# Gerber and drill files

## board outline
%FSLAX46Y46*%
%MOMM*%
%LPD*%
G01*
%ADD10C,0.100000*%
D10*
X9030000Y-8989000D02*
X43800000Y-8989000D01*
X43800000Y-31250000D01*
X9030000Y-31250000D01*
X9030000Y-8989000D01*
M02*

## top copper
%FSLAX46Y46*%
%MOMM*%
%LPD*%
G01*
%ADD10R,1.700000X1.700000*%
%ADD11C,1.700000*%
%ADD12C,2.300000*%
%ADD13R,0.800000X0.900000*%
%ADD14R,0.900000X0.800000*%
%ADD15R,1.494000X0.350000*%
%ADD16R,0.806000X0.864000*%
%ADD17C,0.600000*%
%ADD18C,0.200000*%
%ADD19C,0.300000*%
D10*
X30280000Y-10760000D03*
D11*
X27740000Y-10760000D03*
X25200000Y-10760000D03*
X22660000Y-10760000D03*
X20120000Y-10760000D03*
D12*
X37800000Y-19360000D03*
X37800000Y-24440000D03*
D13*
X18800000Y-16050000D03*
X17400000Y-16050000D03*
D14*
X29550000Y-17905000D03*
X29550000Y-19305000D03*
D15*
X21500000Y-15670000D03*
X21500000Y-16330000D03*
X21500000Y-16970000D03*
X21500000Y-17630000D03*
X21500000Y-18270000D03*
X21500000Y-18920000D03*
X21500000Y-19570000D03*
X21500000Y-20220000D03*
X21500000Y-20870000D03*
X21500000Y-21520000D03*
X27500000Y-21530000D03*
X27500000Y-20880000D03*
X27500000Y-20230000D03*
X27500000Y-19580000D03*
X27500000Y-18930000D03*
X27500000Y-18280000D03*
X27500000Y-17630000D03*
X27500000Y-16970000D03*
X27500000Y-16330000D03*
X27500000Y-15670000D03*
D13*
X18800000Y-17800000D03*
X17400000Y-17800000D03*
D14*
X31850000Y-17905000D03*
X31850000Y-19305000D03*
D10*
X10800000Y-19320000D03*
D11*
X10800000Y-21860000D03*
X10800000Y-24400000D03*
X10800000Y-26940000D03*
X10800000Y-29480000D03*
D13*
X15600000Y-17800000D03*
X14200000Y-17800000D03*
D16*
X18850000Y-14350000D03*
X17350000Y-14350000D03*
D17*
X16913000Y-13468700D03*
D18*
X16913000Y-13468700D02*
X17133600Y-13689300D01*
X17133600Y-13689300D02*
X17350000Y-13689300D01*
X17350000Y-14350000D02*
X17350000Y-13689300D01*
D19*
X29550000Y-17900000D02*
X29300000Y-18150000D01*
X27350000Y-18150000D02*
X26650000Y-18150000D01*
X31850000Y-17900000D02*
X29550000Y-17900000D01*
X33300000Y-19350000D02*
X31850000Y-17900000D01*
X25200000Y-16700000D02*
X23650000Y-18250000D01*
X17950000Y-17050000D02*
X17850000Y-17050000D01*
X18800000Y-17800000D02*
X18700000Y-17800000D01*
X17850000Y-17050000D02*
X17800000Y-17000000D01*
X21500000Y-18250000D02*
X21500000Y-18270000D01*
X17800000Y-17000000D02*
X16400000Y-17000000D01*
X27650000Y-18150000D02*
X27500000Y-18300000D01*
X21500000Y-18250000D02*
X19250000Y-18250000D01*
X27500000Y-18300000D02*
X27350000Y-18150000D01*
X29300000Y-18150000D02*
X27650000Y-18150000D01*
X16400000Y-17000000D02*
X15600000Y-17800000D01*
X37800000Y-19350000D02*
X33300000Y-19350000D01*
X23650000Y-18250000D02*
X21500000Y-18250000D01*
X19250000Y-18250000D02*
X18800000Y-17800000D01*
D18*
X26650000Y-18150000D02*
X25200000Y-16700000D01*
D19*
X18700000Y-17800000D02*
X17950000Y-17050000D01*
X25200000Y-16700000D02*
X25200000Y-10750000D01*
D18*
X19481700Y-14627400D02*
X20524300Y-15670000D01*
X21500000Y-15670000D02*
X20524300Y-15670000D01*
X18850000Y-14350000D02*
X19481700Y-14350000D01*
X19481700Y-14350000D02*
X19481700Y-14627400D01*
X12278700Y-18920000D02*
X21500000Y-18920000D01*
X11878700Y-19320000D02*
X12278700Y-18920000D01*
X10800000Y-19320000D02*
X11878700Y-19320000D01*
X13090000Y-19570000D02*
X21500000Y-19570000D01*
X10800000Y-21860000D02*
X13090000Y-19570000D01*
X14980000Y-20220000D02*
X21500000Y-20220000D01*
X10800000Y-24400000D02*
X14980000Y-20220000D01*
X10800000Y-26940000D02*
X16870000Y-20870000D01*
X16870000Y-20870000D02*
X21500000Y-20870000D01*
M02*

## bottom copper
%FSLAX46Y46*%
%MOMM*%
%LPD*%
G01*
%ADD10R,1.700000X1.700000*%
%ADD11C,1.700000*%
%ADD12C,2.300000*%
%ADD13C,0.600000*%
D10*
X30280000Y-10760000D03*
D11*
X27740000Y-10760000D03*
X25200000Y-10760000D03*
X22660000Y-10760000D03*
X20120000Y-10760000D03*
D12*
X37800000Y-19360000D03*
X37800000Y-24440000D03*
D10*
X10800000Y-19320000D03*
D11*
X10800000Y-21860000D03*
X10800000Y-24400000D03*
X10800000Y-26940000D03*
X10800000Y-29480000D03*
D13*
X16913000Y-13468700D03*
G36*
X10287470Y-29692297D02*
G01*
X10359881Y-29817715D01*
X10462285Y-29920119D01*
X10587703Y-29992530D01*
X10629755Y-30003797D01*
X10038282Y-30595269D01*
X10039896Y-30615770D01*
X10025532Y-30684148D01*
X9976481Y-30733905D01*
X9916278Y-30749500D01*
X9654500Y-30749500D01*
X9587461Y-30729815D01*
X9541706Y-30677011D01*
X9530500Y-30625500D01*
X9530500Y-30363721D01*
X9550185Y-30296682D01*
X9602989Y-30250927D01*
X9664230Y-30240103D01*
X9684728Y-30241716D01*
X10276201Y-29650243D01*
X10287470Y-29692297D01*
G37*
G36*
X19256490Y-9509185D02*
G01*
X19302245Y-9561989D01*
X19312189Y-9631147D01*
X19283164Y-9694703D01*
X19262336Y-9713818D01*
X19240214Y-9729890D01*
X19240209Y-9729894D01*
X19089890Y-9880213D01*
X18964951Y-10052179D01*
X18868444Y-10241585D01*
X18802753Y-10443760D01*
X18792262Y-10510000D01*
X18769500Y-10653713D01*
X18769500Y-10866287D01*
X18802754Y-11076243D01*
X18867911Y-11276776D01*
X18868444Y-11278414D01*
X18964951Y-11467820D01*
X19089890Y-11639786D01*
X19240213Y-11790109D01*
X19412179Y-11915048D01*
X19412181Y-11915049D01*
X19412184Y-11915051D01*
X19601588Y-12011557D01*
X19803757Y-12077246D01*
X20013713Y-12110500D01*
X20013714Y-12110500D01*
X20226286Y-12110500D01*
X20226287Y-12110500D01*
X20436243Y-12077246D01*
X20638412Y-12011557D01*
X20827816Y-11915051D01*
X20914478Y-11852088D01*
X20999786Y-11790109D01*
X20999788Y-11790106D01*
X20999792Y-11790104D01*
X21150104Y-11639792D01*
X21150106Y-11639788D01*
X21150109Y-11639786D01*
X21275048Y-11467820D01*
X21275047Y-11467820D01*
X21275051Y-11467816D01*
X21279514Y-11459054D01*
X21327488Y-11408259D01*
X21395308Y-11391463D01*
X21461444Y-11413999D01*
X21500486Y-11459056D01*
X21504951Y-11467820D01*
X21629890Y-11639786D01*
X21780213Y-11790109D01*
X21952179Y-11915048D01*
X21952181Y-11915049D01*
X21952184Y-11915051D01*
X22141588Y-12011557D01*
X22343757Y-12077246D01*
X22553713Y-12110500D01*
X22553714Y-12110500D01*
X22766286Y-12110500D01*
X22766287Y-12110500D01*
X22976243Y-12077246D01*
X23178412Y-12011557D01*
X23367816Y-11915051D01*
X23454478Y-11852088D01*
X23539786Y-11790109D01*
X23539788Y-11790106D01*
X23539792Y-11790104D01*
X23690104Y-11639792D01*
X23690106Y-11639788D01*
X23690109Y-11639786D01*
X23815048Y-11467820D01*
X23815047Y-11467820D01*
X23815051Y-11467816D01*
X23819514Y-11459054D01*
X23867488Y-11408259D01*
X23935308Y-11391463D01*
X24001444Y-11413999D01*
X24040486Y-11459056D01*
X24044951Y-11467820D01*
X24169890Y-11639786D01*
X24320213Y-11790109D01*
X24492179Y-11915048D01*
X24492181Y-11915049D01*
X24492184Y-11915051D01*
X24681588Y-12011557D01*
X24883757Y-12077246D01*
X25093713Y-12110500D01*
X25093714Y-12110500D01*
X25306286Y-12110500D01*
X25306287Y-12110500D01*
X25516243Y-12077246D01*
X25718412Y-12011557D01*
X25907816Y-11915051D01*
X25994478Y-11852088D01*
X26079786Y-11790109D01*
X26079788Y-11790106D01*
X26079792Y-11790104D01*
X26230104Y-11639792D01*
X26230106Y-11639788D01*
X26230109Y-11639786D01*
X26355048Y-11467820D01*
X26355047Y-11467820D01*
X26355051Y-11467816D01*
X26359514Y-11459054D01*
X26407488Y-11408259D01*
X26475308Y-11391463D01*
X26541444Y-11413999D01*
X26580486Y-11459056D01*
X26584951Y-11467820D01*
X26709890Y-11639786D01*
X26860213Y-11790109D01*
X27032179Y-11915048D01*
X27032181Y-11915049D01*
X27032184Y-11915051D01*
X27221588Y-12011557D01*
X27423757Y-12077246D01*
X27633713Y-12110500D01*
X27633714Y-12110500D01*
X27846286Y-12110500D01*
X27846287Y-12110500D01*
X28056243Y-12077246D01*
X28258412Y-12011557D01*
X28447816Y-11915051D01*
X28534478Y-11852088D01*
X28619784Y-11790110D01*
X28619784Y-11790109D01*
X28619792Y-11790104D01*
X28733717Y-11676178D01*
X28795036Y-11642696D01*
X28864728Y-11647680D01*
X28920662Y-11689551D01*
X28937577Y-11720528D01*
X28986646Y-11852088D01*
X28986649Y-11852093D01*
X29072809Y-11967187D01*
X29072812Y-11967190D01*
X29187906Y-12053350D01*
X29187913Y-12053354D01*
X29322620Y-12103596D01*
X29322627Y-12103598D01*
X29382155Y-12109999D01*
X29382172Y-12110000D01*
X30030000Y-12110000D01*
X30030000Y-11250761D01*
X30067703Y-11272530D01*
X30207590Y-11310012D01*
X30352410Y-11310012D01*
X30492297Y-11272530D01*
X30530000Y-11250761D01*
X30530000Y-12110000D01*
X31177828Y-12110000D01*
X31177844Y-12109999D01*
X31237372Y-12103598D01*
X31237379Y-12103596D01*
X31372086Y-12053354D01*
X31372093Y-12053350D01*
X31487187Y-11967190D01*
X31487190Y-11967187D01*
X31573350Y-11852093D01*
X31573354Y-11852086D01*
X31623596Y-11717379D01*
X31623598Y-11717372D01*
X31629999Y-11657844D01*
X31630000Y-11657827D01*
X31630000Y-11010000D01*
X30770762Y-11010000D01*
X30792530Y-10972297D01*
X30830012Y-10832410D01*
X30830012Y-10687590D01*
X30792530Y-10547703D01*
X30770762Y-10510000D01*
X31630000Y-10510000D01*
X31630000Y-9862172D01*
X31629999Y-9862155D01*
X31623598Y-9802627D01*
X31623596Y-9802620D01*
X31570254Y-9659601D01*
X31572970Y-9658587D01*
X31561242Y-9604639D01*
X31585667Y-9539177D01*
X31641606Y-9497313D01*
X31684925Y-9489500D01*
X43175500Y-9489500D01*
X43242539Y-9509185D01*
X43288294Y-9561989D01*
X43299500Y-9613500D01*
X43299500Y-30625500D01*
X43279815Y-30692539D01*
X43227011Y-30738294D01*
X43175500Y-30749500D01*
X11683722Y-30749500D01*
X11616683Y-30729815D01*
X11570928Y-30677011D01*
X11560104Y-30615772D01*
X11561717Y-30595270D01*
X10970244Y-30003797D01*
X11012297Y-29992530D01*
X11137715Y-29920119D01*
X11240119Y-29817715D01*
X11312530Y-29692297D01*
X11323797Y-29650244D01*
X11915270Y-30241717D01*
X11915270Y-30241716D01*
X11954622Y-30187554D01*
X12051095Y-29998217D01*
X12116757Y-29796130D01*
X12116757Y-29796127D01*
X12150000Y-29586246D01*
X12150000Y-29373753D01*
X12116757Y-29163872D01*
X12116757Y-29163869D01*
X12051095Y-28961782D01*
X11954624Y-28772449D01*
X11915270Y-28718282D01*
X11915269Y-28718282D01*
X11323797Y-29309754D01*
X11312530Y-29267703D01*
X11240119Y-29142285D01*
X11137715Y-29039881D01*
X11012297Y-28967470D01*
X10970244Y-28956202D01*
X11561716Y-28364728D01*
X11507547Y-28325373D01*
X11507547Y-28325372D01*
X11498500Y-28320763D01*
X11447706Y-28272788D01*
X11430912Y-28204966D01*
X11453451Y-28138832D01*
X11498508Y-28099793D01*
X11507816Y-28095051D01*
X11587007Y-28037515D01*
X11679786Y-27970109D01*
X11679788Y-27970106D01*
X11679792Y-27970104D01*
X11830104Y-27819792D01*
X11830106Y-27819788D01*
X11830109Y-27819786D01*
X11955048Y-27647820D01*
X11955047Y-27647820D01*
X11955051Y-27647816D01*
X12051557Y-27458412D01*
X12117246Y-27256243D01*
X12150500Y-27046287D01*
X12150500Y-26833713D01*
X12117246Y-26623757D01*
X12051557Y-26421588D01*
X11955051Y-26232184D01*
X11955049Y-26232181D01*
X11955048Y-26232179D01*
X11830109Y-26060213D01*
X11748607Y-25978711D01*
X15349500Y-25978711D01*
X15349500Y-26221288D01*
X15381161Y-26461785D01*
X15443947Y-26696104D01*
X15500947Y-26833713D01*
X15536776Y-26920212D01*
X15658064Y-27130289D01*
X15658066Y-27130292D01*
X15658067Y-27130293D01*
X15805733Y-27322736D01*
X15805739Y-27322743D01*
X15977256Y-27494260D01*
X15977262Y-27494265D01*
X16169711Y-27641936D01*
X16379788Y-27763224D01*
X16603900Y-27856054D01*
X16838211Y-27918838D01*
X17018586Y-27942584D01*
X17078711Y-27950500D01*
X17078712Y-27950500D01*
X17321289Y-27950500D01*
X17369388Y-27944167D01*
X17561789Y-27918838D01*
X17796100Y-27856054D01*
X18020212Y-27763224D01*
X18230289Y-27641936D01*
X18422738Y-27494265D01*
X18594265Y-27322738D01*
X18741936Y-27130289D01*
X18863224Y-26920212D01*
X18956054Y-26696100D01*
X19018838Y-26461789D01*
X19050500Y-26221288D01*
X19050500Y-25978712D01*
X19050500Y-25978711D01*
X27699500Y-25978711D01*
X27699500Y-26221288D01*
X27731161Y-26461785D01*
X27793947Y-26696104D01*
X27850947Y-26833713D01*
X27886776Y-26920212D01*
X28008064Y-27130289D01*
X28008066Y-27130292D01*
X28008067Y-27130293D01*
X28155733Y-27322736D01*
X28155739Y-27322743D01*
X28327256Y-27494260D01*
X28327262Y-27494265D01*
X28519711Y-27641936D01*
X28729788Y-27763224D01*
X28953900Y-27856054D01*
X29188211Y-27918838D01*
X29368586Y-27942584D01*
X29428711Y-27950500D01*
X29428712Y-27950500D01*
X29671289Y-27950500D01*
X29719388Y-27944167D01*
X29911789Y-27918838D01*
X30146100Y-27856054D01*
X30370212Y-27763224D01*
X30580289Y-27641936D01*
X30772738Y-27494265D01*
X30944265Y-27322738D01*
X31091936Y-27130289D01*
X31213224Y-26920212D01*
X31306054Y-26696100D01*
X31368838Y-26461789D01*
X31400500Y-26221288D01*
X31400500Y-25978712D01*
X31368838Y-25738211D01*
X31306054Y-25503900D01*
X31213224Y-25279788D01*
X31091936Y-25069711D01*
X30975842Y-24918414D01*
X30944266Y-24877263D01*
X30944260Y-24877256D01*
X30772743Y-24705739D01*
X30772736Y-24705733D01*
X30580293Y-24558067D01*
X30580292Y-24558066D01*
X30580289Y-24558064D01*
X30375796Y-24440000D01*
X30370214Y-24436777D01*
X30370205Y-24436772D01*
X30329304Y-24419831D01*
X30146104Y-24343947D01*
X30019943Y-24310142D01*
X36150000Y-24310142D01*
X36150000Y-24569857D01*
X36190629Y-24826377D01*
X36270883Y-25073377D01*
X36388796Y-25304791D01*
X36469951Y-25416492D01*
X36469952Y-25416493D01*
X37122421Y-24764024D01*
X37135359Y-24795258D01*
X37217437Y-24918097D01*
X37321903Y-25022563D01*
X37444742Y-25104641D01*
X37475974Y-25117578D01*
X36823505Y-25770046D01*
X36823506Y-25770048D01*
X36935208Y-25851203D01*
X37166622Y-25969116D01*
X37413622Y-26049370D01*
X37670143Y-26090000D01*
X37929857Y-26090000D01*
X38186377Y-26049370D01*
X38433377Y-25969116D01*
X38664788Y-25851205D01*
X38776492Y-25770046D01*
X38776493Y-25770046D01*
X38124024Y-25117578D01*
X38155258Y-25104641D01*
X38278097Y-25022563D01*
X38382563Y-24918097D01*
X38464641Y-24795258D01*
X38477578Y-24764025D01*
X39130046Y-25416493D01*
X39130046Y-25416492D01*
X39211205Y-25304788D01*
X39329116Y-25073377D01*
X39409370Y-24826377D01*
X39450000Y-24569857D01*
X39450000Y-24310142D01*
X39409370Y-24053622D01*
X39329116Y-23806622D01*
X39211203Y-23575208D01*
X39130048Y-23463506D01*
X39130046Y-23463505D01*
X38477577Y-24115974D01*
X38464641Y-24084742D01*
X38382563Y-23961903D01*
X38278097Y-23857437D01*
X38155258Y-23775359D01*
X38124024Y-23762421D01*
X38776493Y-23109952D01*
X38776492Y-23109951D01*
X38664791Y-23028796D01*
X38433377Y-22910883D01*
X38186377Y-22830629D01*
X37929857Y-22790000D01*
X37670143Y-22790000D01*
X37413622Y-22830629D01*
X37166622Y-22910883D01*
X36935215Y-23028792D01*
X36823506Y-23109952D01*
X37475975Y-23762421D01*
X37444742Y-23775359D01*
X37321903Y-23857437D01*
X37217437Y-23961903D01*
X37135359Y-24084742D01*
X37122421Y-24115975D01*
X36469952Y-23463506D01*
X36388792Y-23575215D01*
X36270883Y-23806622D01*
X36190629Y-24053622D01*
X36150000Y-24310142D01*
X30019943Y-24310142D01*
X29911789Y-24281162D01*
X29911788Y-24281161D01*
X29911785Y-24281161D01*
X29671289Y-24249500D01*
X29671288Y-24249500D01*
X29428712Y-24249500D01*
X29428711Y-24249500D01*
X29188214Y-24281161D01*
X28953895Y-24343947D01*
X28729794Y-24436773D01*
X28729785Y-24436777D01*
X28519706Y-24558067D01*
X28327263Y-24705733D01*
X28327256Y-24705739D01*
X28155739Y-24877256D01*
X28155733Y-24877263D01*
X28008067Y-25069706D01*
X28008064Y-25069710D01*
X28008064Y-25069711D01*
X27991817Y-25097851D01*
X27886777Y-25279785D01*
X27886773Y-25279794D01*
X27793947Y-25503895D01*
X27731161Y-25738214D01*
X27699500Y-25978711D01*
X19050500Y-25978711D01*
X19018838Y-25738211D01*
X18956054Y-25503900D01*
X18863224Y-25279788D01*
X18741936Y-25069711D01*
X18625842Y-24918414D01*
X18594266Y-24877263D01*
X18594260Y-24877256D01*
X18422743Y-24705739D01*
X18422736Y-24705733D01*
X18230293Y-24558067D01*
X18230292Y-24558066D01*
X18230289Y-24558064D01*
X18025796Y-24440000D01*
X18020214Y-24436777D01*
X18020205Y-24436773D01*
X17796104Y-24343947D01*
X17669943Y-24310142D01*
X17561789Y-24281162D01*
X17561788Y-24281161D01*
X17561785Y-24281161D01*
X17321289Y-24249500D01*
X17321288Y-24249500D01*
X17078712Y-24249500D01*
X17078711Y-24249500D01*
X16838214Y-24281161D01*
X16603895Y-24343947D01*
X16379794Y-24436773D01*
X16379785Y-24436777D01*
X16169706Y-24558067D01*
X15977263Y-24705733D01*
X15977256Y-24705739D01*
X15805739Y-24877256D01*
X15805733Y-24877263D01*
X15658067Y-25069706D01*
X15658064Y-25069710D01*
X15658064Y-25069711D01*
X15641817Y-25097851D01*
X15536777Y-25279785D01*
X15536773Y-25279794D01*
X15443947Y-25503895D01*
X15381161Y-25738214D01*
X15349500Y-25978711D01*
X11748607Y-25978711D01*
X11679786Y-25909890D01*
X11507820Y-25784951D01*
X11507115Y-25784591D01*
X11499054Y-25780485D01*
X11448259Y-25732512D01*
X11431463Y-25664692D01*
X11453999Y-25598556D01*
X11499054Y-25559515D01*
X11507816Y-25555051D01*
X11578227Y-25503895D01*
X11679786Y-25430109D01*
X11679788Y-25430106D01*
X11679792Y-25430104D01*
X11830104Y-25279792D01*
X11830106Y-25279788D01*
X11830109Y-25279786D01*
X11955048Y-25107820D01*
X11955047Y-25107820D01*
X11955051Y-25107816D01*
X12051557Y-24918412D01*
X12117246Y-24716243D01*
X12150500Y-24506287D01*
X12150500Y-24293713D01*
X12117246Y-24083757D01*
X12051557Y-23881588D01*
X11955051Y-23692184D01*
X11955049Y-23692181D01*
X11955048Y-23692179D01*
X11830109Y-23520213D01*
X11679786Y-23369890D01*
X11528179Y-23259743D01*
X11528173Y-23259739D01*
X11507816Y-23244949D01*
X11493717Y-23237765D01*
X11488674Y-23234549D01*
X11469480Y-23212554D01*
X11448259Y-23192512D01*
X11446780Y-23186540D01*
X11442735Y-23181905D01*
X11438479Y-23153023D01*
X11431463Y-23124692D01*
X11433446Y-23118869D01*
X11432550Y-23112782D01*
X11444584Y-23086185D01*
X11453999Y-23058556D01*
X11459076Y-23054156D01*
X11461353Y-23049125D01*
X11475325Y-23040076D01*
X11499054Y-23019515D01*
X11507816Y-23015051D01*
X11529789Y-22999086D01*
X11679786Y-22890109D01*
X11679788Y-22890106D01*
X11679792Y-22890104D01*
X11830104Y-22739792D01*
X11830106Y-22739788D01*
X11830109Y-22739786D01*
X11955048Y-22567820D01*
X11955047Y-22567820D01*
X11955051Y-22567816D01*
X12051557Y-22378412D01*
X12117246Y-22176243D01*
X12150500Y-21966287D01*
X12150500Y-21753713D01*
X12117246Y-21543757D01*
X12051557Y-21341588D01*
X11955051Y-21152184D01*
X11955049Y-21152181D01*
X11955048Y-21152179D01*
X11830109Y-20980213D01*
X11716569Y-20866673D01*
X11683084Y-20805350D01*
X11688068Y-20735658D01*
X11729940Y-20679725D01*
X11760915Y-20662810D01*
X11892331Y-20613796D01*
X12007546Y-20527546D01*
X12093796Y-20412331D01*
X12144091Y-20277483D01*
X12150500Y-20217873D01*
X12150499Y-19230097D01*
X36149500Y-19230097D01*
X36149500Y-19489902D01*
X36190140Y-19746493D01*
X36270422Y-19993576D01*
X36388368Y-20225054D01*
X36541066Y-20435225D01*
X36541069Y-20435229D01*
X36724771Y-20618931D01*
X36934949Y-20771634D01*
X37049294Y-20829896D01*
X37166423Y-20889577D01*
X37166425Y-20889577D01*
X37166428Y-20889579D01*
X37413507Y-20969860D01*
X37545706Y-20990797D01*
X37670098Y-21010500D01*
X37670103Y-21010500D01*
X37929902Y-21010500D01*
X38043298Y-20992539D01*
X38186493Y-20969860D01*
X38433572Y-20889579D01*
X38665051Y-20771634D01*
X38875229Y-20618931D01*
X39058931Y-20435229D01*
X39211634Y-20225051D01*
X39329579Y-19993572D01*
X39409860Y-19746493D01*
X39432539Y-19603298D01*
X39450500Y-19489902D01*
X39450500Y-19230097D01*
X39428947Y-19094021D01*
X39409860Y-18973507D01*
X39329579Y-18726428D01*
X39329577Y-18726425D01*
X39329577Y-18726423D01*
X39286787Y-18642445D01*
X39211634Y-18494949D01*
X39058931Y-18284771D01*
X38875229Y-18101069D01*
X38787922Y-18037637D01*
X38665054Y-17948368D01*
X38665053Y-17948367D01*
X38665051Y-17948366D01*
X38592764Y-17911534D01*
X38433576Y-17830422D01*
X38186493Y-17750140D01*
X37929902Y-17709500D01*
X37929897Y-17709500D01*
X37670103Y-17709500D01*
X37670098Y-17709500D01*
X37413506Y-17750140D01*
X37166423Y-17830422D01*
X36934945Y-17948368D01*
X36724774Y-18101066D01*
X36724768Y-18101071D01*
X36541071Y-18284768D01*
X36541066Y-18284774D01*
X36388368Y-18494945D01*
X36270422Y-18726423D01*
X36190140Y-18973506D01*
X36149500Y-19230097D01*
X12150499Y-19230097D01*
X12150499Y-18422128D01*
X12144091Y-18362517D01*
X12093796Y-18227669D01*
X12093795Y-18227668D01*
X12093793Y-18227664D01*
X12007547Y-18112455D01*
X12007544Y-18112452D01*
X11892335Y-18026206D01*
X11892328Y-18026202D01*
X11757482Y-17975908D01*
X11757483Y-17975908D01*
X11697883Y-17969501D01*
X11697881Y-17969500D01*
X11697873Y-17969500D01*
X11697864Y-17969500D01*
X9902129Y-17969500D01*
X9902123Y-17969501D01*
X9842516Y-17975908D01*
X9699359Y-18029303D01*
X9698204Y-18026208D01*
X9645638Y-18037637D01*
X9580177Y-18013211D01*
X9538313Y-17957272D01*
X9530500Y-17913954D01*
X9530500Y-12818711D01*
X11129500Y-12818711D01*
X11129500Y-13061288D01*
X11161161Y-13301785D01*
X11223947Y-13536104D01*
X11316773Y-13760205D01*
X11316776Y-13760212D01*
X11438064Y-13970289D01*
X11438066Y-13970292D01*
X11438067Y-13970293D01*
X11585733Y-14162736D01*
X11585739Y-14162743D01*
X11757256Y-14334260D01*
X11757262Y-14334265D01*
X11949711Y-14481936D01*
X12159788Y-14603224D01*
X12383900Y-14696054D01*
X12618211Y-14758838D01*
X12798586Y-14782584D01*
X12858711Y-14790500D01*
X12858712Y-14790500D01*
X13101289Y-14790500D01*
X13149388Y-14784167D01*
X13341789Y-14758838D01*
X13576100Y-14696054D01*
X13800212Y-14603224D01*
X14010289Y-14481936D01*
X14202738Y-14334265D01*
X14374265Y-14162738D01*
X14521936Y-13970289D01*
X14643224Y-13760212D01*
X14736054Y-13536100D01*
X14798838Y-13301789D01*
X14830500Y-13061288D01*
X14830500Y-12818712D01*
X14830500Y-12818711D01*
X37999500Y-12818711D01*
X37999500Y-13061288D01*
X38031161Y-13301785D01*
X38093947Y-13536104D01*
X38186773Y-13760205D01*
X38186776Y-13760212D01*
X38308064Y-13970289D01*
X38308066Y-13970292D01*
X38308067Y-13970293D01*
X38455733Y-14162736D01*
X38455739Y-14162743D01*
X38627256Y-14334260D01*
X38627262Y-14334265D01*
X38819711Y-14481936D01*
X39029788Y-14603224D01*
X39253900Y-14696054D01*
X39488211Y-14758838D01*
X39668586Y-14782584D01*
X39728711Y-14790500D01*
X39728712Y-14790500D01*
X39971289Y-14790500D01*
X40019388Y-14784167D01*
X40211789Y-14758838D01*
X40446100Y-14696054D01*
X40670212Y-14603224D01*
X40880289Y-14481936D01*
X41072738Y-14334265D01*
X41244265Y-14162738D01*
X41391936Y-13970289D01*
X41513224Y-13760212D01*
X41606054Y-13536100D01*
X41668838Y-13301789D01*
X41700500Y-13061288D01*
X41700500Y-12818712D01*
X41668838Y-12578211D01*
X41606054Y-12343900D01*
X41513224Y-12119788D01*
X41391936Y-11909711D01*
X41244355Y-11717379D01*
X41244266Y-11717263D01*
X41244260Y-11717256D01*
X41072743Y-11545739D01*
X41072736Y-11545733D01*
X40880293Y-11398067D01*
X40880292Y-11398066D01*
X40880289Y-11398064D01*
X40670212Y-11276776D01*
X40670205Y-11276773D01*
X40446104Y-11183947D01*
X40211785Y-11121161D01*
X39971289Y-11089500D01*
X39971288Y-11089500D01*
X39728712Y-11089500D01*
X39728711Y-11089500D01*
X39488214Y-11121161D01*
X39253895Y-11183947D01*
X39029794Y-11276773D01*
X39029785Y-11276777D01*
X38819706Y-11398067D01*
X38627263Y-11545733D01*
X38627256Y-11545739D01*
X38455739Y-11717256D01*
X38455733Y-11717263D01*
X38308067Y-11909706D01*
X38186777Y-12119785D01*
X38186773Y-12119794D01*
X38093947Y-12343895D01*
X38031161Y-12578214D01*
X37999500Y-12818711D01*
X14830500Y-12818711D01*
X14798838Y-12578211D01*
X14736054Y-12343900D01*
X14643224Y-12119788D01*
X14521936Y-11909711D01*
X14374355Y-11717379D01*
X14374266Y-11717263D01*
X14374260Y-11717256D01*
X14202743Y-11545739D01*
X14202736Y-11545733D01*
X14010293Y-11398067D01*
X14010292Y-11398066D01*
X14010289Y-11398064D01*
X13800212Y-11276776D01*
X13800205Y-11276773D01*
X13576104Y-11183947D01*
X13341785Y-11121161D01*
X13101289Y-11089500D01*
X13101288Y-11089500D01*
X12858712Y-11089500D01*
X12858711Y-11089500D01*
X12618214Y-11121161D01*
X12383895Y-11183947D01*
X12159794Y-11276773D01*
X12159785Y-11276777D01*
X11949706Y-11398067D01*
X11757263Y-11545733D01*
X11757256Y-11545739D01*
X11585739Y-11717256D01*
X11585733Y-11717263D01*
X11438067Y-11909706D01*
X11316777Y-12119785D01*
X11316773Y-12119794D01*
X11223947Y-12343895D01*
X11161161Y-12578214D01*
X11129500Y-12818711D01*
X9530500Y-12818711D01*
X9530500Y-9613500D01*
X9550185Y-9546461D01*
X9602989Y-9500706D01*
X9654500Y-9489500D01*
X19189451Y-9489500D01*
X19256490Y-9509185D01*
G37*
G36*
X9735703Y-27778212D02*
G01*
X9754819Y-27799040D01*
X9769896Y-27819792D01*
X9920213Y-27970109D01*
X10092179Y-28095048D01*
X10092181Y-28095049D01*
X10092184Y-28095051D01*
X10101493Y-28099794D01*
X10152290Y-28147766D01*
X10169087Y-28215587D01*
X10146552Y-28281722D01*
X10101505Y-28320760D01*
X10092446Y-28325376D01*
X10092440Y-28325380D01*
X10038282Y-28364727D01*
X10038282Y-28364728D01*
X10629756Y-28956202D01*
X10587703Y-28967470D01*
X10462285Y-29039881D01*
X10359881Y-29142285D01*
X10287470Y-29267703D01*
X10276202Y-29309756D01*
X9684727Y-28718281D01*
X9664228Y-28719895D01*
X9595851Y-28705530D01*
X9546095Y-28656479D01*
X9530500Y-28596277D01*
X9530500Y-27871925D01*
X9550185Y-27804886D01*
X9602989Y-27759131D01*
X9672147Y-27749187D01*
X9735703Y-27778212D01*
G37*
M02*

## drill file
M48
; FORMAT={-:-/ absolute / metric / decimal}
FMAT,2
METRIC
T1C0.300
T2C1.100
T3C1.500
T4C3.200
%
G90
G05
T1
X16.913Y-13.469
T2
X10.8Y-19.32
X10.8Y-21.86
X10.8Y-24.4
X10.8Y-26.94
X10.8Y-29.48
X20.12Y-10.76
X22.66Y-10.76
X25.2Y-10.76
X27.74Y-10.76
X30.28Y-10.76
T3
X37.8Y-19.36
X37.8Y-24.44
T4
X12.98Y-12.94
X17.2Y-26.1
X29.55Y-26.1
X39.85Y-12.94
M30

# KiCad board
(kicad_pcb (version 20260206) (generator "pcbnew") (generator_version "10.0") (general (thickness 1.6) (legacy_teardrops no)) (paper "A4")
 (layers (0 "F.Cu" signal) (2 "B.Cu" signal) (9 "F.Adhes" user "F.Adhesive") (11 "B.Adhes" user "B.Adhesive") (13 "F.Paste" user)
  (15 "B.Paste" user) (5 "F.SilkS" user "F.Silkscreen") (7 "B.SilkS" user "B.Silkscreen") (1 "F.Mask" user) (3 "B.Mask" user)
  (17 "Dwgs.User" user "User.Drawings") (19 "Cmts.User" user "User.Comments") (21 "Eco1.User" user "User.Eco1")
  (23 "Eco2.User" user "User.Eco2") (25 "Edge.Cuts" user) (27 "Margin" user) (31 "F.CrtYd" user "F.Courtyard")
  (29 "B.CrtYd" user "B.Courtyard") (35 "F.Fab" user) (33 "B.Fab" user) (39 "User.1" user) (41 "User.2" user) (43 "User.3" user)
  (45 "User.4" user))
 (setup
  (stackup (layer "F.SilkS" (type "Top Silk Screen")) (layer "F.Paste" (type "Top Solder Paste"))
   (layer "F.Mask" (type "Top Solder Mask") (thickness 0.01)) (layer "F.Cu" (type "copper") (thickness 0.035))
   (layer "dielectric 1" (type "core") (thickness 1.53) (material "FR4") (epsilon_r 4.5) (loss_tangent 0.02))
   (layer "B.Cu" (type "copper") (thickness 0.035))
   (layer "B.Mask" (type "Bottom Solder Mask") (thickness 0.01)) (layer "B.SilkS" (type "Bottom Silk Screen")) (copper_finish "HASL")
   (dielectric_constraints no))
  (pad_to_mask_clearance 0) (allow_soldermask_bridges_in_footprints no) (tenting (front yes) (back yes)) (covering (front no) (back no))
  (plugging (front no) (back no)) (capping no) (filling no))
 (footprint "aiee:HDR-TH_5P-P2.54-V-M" (layer "F.Cu") (at 25.2 10.76 180)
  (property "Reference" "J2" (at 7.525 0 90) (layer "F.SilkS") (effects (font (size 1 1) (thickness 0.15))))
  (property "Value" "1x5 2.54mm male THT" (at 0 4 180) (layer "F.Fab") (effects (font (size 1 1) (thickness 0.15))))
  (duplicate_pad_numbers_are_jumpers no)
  (pad "1" thru_hole rect (at -5.08 0 180) (size 1.7 1.7) (drill 1.100024) (layers "*.Cu" "*.Mask") (remove_unused_layers no) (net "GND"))
  (pad "2" thru_hole circle (at -2.54 0 180) (size 1.7 1.7) (drill 1.100024) (layers "*.Cu" "*.Mask") (remove_unused_layers no)
   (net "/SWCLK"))
  (pad "3" thru_hole circle (at 0 0 180) (size 1.7 1.7) (drill 1.100024) (layers "*.Cu" "*.Mask") (remove_unused_layers no) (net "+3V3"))
  (pad "4" thru_hole circle (at 2.54 0 180) (size 1.7 1.7) (drill 1.100024) (layers "*.Cu" "*.Mask") (remove_unused_layers no)
   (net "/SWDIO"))
  (pad "5" thru_hole circle (at 5.08 0 180) (size 1.7 1.7) (drill 1.100024) (layers "*.Cu" "*.Mask") (remove_unused_layers no) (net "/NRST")))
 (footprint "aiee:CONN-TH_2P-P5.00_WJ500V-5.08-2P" (layer "F.Cu") (at 37.8 21.9 -90)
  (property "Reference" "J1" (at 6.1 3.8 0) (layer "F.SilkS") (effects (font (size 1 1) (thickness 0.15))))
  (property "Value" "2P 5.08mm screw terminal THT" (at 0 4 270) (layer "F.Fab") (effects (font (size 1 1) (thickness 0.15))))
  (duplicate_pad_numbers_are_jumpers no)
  (pad "1" thru_hole circle (at -2.54 0 90) (size 2.3 2.3) (drill 1.5) (layers "*.Cu" "*.Mask") (remove_unused_layers no) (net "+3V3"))
  (pad "2" thru_hole circle (at 2.54 0 90) (size 2.3 2.3) (drill 1.5) (layers "*.Cu" "*.Mask") (remove_unused_layers no) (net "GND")))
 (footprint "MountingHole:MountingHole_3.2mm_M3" (layer "F.Cu") (at 29.55 26.1)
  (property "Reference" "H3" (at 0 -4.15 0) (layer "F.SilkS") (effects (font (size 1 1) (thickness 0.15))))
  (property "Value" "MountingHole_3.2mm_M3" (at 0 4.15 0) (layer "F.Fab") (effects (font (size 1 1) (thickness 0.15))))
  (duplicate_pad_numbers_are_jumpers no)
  (pad "" np_thru_hole circle (at 0 0) (size 3.2 3.2) (drill 3.2) (layers "*.Cu" "*.Mask")))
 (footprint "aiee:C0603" (layer "F.Cu") (at 18.1 16.05 180)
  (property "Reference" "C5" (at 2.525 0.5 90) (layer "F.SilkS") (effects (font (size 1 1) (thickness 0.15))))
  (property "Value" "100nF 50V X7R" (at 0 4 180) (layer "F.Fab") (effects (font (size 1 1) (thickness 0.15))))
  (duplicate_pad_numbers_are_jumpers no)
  (pad "1" smd rect (at -0.7 0 180) (size 0.8 0.9) (layers "F.Cu" "F.Mask" "F.Paste") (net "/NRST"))
  (pad "2" smd rect (at 0.7 0 180) (size 0.8 0.9) (layers "F.Cu" "F.Mask" "F.Paste") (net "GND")))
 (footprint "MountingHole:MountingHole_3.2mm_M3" (layer "F.Cu") (at 17.2 26.1)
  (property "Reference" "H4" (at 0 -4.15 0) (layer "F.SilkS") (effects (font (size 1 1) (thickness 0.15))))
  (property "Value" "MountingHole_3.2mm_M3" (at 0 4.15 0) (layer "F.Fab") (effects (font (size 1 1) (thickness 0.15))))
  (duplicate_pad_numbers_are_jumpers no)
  (pad "" np_thru_hole circle (at 0 0) (size 3.2 3.2) (drill 3.2) (layers "*.Cu" "*.Mask")))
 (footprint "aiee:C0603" (layer "F.Cu") (at 29.55 18.605 -90)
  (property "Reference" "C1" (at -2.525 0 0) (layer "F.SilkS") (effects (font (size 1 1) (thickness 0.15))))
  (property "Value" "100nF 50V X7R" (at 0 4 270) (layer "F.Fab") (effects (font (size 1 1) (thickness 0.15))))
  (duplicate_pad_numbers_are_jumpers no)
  (pad "1" smd rect (at -0.7 0 270) (size 0.8 0.9) (layers "F.Cu" "F.Mask" "F.Paste") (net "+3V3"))
  (pad "2" smd rect (at 0.7 0 270) (size 0.8 0.9) (layers "F.Cu" "F.Mask" "F.Paste") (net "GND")))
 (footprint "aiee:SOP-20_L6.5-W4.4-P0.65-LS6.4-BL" (layer "F.Cu") (at 24.5 18.6 -90)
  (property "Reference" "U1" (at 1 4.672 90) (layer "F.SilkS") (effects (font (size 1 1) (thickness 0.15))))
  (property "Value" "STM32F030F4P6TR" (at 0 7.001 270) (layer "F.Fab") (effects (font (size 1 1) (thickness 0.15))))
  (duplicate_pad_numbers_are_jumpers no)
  (pad "1" smd rect (at -2.93 3 270) (size 0.35 1.494) (layers "F.Cu" "F.Mask" "F.Paste") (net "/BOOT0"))
  (pad "2" smd rect (at -2.27 3 270) (size 0.35 1.494) (layers "F.Cu" "F.Mask" "F.Paste") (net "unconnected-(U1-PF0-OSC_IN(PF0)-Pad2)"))
  (pad "3" smd rect (at -1.63 3 270) (size 0.35 1.494) (layers "F.Cu" "F.Mask" "F.Paste") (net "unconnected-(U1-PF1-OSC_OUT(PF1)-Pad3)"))
  (pad "4" smd rect (at -0.97 3 270) (size 0.35 1.494) (layers "F.Cu" "F.Mask" "F.Paste") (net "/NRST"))
  (pad "5" smd rect (at -0.33 3 270) (size 0.35 1.494) (layers "F.Cu" "F.Mask" "F.Paste") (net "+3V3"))
  (pad "6" smd rect (at 0.32 3 270) (size 0.35 1.494) (layers "F.Cu" "F.Mask" "F.Paste") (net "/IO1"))
  (pad "7" smd rect (at 0.97 3 270) (size 0.35 1.494) (layers "F.Cu" "F.Mask" "F.Paste") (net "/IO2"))
  (pad "8" smd rect (at 1.62 3 270) (size 0.35 1.494) (layers "F.Cu" "F.Mask" "F.Paste") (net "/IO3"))
  (pad "9" smd rect (at 2.27 3 270) (size 0.35 1.494) (layers "F.Cu" "F.Mask" "F.Paste") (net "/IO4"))
  (pad "10" smd rect (at 2.92 3 270) (size 0.35 1.494) (layers "F.Cu" "F.Mask" "F.Paste") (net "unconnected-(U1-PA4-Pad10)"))
  (pad "11" smd rect (at 2.93 -3 270) (size 0.35 1.494) (layers "F.Cu" "F.Mask" "F.Paste") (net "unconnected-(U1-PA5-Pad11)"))
  (pad "12" smd rect (at 2.28 -3 270) (size 0.35 1.494) (layers "F.Cu" "F.Mask" "F.Paste") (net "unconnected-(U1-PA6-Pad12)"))
  (pad "13" smd rect (at 1.63 -3 270) (size 0.35 1.494) (layers "F.Cu" "F.Mask" "F.Paste") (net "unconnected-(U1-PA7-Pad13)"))
  (pad "14" smd rect (at 0.98 -3 270) (size 0.35 1.494) (layers "F.Cu" "F.Mask" "F.Paste") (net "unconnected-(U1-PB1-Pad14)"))
  (pad "15" smd rect (at 0.33 -3 270) (size 0.35 1.494) (layers "F.Cu" "F.Mask" "F.Paste") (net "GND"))
  (pad "16" smd rect (at -0.32 -3 270) (size 0.35 1.494) (layers "F.Cu" "F.Mask" "F.Paste") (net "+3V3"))
  (pad "17" smd rect (at -0.97 -3 270) (size 0.35 1.494) (layers "F.Cu" "F.Mask" "F.Paste") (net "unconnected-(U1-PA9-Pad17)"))
  (pad "18" smd rect (at -1.63 -3 270) (size 0.35 1.494) (layers "F.Cu" "F.Mask" "F.Paste") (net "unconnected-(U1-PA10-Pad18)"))
  (pad "19" smd rect (at -2.27 -3 270) (size 0.35 1.494) (layers "F.Cu" "F.Mask" "F.Paste") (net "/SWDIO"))
  (pad "20" smd rect (at -2.93 -3 270) (size 0.35 1.494) (layers "F.Cu" "F.Mask" "F.Paste") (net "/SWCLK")))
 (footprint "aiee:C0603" (layer "F.Cu") (at 18.1 17.8 180)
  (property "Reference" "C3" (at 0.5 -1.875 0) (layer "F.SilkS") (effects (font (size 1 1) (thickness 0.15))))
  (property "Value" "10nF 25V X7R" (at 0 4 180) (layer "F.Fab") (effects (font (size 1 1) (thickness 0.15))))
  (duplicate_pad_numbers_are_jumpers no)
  (pad "1" smd rect (at -0.7 0 180) (size 0.8 0.9) (layers "F.Cu" "F.Mask" "F.Paste") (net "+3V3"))
  (pad "2" smd rect (at 0.7 0 180) (size 0.8 0.9) (layers "F.Cu" "F.Mask" "F.Paste") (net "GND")))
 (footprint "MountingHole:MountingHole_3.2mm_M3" (layer "F.Cu") (at 12.98 12.94)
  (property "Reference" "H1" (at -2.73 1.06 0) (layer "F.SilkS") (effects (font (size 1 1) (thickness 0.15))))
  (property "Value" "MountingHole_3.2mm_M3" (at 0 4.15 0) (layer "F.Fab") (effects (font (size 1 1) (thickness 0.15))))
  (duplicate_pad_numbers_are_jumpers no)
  (pad "" np_thru_hole circle (at 0 0) (size 3.2 3.2) (drill 3.2) (layers "*.Cu" "*.Mask")))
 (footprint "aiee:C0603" (layer "F.Cu") (at 31.85 18.605 -90)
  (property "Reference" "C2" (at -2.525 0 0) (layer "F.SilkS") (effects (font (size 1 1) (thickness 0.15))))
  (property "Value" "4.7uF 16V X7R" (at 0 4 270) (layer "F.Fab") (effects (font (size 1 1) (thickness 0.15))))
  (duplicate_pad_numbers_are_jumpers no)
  (pad "1" smd rect (at -0.7 0 270) (size 0.8 0.9) (layers "F.Cu" "F.Mask" "F.Paste") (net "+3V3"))
  (pad "2" smd rect (at 0.7 0 270) (size 0.8 0.9) (layers "F.Cu" "F.Mask" "F.Paste") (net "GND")))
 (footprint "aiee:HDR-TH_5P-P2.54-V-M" (layer "F.Cu") (at 10.8 24.4 -90)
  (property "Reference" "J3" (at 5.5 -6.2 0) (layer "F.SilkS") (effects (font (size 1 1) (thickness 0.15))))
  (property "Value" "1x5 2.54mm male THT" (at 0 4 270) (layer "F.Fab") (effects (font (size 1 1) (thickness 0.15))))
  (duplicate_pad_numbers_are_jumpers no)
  (pad "1" thru_hole rect (at -5.08 0 270) (size 1.7 1.7) (drill 1.100024) (layers "*.Cu" "*.Mask") (remove_unused_layers no) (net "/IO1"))
  (pad "2" thru_hole circle (at -2.54 0 270) (size 1.7 1.7) (drill 1.100024) (layers "*.Cu" "*.Mask") (remove_unused_layers no) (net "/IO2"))
  (pad "3" thru_hole circle (at 0 0 270) (size 1.7 1.7) (drill 1.100024) (layers "*.Cu" "*.Mask") (remove_unused_layers no) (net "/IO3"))
  (pad "4" thru_hole circle (at 2.54 0 270) (size 1.7 1.7) (drill 1.100024) (layers "*.Cu" "*.Mask") (remove_unused_layers no) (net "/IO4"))
  (pad "5" thru_hole circle (at 5.08 0 270) (size 1.7 1.7) (drill 1.100024) (layers "*.Cu" "*.Mask") (remove_unused_layers no) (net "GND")))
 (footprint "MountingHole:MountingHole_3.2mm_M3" (layer "F.Cu") (at 39.85 12.94)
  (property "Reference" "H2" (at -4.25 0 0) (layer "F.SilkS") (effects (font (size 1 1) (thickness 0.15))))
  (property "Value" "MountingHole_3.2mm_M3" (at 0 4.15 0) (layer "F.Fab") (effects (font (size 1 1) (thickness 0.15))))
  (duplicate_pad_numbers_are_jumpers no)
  (pad "" np_thru_hole circle (at 0 0) (size 3.2 3.2) (drill 3.2) (layers "*.Cu" "*.Mask")))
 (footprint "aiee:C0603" (layer "F.Cu") (at 14.9 17.8 180)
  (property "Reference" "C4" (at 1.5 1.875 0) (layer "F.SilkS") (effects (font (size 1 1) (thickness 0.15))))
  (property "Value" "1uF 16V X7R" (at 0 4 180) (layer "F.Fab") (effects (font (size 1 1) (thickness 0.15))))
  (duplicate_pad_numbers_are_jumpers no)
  (pad "1" smd rect (at -0.7 0 180) (size 0.8 0.9) (layers "F.Cu" "F.Mask" "F.Paste") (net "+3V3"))
  (pad "2" smd rect (at 0.7 0 180) (size 0.8 0.9) (layers "F.Cu" "F.Mask" "F.Paste") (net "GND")))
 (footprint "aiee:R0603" (layer "F.Cu") (at 18.1 14.35 180)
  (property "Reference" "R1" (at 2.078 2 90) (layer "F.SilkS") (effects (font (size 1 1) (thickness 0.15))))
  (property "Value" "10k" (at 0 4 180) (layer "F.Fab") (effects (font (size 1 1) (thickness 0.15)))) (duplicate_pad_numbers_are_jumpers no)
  (pad "1" smd rect (at -0.75 0 180) (size 0.806 0.864) (layers "F.Cu" "F.Mask" "F.Paste") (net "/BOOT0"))
  (pad "2" smd rect (at 0.75 0 180) (size 0.806 0.864) (layers "F.Cu" "F.Mask" "F.Paste") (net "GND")))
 (gr_rect (start 9.03 8.989) (end 43.8 31.25) (stroke (width 0.1) (type default)) (fill no) (layer "Edge.Cuts"))
 (segment (start 16.913 13.4687) (end 17.1336 13.6893) (width 0.2) (layer "F.Cu") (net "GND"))
 (segment (start 17.1336 13.6893) (end 17.35 13.6893) (width 0.2) (layer "F.Cu") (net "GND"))
 (segment (start 17.35 14.35) (end 17.35 13.6893) (width 0.2) (layer "F.Cu") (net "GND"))
 (via (at 16.913 13.4687) (size 0.6) (drill 0.3) (layers "F.Cu" "B.Cu") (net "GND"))
 (segment (start 29.55 17.9) (end 29.3 18.15) (width 0.3) (layer "F.Cu") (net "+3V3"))
 (segment (start 27.35 18.15) (end 26.65 18.15) (width 0.3) (layer "F.Cu") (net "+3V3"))
 (segment (start 31.85 17.9) (end 29.55 17.9) (width 0.3) (layer "F.Cu") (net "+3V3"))
 (segment (start 33.3 19.35) (end 31.85 17.9) (width 0.3) (layer "F.Cu") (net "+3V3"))
 (segment (start 25.2 16.7) (end 23.65 18.25) (width 0.3) (layer "F.Cu") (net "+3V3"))
 (segment (start 17.95 17.05) (end 17.85 17.05) (width 0.3) (layer "F.Cu") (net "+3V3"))
 (segment (start 18.8 17.8) (end 18.7 17.8) (width 0.3) (layer "F.Cu") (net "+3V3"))
 (segment (start 17.85 17.05) (end 17.8 17) (width 0.3) (layer "F.Cu") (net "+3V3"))
 (segment (start 21.5 18.25) (end 21.5 18.27) (width 0.3) (layer "F.Cu") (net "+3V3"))
 (segment (start 17.8 17) (end 16.4 17) (width 0.3) (layer "F.Cu") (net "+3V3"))
 (segment (start 27.65 18.15) (end 27.5 18.3) (width 0.3) (layer "F.Cu") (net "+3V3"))
 (segment (start 21.5 18.25) (end 19.25 18.25) (width 0.3) (layer "F.Cu") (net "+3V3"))
 (segment (start 27.5 18.3) (end 27.35 18.15) (width 0.3) (layer "F.Cu") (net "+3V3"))
 (segment (start 29.3 18.15) (end 27.65 18.15) (width 0.3) (layer "F.Cu") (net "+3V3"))
 (segment (start 16.4 17) (end 15.6 17.8) (width 0.3) (layer "F.Cu") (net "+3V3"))
 (segment (start 37.8 19.35) (end 33.3 19.35) (width 0.3) (layer "F.Cu") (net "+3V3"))
 (segment (start 23.65 18.25) (end 21.5 18.25) (width 0.3) (layer "F.Cu") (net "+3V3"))
 (segment (start 19.25 18.25) (end 18.8 17.8) (width 0.3) (layer "F.Cu") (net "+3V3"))
 (segment (start 26.65 18.15) (end 25.2 16.7) (width 0.2) (layer "F.Cu") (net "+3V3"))
 (segment (start 18.7 17.8) (end 17.95 17.05) (width 0.3) (layer "F.Cu") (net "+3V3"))
 (segment (start 25.2 16.7) (end 25.2 10.75) (width 0.3) (layer "F.Cu") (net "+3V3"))
 (segment (start 19.4817 14.6274) (end 20.5243 15.67) (width 0.2) (layer "F.Cu") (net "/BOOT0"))
 (segment (start 21.5 15.67) (end 20.5243 15.67) (width 0.2) (layer "F.Cu") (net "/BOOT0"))
 (segment (start 18.85 14.35) (end 19.4817 14.35) (width 0.2) (layer "F.Cu") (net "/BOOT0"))
 (segment (start 19.4817 14.35) (end 19.4817 14.6274) (width 0.2) (layer "F.Cu") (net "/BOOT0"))
 (segment (start 12.2787 18.92) (end 21.5 18.92) (width 0.2) (layer "F.Cu") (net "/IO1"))
 (segment (start 11.8787 19.32) (end 12.2787 18.92) (width 0.2) (layer "F.Cu") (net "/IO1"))
 (segment (start 10.8 19.32) (end 11.8787 19.32) (width 0.2) (layer "F.Cu") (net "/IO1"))
 (segment (start 13.09 19.57) (end 21.5 19.57) (width 0.2) (layer "F.Cu") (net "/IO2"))
 (segment (start 10.8 21.86) (end 13.09 19.57) (width 0.2) (layer "F.Cu") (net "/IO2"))
 (segment (start 14.98 20.22) (end 21.5 20.22) (width 0.2) (layer "F.Cu") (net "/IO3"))
 (segment (start 10.8 24.4) (end 14.98 20.22) (width 0.2) (layer "F.Cu") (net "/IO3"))
 (segment (start 10.8 26.94) (end 16.87 20.87) (width 0.2) (layer "F.Cu") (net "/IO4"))
 (segment (start 16.87 20.87) (end 21.5 20.87) (width 0.2) (layer "F.Cu") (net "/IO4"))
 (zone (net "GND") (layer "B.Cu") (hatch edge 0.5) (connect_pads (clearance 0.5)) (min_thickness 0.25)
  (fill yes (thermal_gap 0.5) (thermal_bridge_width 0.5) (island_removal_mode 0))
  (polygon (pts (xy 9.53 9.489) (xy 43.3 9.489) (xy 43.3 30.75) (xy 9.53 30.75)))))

